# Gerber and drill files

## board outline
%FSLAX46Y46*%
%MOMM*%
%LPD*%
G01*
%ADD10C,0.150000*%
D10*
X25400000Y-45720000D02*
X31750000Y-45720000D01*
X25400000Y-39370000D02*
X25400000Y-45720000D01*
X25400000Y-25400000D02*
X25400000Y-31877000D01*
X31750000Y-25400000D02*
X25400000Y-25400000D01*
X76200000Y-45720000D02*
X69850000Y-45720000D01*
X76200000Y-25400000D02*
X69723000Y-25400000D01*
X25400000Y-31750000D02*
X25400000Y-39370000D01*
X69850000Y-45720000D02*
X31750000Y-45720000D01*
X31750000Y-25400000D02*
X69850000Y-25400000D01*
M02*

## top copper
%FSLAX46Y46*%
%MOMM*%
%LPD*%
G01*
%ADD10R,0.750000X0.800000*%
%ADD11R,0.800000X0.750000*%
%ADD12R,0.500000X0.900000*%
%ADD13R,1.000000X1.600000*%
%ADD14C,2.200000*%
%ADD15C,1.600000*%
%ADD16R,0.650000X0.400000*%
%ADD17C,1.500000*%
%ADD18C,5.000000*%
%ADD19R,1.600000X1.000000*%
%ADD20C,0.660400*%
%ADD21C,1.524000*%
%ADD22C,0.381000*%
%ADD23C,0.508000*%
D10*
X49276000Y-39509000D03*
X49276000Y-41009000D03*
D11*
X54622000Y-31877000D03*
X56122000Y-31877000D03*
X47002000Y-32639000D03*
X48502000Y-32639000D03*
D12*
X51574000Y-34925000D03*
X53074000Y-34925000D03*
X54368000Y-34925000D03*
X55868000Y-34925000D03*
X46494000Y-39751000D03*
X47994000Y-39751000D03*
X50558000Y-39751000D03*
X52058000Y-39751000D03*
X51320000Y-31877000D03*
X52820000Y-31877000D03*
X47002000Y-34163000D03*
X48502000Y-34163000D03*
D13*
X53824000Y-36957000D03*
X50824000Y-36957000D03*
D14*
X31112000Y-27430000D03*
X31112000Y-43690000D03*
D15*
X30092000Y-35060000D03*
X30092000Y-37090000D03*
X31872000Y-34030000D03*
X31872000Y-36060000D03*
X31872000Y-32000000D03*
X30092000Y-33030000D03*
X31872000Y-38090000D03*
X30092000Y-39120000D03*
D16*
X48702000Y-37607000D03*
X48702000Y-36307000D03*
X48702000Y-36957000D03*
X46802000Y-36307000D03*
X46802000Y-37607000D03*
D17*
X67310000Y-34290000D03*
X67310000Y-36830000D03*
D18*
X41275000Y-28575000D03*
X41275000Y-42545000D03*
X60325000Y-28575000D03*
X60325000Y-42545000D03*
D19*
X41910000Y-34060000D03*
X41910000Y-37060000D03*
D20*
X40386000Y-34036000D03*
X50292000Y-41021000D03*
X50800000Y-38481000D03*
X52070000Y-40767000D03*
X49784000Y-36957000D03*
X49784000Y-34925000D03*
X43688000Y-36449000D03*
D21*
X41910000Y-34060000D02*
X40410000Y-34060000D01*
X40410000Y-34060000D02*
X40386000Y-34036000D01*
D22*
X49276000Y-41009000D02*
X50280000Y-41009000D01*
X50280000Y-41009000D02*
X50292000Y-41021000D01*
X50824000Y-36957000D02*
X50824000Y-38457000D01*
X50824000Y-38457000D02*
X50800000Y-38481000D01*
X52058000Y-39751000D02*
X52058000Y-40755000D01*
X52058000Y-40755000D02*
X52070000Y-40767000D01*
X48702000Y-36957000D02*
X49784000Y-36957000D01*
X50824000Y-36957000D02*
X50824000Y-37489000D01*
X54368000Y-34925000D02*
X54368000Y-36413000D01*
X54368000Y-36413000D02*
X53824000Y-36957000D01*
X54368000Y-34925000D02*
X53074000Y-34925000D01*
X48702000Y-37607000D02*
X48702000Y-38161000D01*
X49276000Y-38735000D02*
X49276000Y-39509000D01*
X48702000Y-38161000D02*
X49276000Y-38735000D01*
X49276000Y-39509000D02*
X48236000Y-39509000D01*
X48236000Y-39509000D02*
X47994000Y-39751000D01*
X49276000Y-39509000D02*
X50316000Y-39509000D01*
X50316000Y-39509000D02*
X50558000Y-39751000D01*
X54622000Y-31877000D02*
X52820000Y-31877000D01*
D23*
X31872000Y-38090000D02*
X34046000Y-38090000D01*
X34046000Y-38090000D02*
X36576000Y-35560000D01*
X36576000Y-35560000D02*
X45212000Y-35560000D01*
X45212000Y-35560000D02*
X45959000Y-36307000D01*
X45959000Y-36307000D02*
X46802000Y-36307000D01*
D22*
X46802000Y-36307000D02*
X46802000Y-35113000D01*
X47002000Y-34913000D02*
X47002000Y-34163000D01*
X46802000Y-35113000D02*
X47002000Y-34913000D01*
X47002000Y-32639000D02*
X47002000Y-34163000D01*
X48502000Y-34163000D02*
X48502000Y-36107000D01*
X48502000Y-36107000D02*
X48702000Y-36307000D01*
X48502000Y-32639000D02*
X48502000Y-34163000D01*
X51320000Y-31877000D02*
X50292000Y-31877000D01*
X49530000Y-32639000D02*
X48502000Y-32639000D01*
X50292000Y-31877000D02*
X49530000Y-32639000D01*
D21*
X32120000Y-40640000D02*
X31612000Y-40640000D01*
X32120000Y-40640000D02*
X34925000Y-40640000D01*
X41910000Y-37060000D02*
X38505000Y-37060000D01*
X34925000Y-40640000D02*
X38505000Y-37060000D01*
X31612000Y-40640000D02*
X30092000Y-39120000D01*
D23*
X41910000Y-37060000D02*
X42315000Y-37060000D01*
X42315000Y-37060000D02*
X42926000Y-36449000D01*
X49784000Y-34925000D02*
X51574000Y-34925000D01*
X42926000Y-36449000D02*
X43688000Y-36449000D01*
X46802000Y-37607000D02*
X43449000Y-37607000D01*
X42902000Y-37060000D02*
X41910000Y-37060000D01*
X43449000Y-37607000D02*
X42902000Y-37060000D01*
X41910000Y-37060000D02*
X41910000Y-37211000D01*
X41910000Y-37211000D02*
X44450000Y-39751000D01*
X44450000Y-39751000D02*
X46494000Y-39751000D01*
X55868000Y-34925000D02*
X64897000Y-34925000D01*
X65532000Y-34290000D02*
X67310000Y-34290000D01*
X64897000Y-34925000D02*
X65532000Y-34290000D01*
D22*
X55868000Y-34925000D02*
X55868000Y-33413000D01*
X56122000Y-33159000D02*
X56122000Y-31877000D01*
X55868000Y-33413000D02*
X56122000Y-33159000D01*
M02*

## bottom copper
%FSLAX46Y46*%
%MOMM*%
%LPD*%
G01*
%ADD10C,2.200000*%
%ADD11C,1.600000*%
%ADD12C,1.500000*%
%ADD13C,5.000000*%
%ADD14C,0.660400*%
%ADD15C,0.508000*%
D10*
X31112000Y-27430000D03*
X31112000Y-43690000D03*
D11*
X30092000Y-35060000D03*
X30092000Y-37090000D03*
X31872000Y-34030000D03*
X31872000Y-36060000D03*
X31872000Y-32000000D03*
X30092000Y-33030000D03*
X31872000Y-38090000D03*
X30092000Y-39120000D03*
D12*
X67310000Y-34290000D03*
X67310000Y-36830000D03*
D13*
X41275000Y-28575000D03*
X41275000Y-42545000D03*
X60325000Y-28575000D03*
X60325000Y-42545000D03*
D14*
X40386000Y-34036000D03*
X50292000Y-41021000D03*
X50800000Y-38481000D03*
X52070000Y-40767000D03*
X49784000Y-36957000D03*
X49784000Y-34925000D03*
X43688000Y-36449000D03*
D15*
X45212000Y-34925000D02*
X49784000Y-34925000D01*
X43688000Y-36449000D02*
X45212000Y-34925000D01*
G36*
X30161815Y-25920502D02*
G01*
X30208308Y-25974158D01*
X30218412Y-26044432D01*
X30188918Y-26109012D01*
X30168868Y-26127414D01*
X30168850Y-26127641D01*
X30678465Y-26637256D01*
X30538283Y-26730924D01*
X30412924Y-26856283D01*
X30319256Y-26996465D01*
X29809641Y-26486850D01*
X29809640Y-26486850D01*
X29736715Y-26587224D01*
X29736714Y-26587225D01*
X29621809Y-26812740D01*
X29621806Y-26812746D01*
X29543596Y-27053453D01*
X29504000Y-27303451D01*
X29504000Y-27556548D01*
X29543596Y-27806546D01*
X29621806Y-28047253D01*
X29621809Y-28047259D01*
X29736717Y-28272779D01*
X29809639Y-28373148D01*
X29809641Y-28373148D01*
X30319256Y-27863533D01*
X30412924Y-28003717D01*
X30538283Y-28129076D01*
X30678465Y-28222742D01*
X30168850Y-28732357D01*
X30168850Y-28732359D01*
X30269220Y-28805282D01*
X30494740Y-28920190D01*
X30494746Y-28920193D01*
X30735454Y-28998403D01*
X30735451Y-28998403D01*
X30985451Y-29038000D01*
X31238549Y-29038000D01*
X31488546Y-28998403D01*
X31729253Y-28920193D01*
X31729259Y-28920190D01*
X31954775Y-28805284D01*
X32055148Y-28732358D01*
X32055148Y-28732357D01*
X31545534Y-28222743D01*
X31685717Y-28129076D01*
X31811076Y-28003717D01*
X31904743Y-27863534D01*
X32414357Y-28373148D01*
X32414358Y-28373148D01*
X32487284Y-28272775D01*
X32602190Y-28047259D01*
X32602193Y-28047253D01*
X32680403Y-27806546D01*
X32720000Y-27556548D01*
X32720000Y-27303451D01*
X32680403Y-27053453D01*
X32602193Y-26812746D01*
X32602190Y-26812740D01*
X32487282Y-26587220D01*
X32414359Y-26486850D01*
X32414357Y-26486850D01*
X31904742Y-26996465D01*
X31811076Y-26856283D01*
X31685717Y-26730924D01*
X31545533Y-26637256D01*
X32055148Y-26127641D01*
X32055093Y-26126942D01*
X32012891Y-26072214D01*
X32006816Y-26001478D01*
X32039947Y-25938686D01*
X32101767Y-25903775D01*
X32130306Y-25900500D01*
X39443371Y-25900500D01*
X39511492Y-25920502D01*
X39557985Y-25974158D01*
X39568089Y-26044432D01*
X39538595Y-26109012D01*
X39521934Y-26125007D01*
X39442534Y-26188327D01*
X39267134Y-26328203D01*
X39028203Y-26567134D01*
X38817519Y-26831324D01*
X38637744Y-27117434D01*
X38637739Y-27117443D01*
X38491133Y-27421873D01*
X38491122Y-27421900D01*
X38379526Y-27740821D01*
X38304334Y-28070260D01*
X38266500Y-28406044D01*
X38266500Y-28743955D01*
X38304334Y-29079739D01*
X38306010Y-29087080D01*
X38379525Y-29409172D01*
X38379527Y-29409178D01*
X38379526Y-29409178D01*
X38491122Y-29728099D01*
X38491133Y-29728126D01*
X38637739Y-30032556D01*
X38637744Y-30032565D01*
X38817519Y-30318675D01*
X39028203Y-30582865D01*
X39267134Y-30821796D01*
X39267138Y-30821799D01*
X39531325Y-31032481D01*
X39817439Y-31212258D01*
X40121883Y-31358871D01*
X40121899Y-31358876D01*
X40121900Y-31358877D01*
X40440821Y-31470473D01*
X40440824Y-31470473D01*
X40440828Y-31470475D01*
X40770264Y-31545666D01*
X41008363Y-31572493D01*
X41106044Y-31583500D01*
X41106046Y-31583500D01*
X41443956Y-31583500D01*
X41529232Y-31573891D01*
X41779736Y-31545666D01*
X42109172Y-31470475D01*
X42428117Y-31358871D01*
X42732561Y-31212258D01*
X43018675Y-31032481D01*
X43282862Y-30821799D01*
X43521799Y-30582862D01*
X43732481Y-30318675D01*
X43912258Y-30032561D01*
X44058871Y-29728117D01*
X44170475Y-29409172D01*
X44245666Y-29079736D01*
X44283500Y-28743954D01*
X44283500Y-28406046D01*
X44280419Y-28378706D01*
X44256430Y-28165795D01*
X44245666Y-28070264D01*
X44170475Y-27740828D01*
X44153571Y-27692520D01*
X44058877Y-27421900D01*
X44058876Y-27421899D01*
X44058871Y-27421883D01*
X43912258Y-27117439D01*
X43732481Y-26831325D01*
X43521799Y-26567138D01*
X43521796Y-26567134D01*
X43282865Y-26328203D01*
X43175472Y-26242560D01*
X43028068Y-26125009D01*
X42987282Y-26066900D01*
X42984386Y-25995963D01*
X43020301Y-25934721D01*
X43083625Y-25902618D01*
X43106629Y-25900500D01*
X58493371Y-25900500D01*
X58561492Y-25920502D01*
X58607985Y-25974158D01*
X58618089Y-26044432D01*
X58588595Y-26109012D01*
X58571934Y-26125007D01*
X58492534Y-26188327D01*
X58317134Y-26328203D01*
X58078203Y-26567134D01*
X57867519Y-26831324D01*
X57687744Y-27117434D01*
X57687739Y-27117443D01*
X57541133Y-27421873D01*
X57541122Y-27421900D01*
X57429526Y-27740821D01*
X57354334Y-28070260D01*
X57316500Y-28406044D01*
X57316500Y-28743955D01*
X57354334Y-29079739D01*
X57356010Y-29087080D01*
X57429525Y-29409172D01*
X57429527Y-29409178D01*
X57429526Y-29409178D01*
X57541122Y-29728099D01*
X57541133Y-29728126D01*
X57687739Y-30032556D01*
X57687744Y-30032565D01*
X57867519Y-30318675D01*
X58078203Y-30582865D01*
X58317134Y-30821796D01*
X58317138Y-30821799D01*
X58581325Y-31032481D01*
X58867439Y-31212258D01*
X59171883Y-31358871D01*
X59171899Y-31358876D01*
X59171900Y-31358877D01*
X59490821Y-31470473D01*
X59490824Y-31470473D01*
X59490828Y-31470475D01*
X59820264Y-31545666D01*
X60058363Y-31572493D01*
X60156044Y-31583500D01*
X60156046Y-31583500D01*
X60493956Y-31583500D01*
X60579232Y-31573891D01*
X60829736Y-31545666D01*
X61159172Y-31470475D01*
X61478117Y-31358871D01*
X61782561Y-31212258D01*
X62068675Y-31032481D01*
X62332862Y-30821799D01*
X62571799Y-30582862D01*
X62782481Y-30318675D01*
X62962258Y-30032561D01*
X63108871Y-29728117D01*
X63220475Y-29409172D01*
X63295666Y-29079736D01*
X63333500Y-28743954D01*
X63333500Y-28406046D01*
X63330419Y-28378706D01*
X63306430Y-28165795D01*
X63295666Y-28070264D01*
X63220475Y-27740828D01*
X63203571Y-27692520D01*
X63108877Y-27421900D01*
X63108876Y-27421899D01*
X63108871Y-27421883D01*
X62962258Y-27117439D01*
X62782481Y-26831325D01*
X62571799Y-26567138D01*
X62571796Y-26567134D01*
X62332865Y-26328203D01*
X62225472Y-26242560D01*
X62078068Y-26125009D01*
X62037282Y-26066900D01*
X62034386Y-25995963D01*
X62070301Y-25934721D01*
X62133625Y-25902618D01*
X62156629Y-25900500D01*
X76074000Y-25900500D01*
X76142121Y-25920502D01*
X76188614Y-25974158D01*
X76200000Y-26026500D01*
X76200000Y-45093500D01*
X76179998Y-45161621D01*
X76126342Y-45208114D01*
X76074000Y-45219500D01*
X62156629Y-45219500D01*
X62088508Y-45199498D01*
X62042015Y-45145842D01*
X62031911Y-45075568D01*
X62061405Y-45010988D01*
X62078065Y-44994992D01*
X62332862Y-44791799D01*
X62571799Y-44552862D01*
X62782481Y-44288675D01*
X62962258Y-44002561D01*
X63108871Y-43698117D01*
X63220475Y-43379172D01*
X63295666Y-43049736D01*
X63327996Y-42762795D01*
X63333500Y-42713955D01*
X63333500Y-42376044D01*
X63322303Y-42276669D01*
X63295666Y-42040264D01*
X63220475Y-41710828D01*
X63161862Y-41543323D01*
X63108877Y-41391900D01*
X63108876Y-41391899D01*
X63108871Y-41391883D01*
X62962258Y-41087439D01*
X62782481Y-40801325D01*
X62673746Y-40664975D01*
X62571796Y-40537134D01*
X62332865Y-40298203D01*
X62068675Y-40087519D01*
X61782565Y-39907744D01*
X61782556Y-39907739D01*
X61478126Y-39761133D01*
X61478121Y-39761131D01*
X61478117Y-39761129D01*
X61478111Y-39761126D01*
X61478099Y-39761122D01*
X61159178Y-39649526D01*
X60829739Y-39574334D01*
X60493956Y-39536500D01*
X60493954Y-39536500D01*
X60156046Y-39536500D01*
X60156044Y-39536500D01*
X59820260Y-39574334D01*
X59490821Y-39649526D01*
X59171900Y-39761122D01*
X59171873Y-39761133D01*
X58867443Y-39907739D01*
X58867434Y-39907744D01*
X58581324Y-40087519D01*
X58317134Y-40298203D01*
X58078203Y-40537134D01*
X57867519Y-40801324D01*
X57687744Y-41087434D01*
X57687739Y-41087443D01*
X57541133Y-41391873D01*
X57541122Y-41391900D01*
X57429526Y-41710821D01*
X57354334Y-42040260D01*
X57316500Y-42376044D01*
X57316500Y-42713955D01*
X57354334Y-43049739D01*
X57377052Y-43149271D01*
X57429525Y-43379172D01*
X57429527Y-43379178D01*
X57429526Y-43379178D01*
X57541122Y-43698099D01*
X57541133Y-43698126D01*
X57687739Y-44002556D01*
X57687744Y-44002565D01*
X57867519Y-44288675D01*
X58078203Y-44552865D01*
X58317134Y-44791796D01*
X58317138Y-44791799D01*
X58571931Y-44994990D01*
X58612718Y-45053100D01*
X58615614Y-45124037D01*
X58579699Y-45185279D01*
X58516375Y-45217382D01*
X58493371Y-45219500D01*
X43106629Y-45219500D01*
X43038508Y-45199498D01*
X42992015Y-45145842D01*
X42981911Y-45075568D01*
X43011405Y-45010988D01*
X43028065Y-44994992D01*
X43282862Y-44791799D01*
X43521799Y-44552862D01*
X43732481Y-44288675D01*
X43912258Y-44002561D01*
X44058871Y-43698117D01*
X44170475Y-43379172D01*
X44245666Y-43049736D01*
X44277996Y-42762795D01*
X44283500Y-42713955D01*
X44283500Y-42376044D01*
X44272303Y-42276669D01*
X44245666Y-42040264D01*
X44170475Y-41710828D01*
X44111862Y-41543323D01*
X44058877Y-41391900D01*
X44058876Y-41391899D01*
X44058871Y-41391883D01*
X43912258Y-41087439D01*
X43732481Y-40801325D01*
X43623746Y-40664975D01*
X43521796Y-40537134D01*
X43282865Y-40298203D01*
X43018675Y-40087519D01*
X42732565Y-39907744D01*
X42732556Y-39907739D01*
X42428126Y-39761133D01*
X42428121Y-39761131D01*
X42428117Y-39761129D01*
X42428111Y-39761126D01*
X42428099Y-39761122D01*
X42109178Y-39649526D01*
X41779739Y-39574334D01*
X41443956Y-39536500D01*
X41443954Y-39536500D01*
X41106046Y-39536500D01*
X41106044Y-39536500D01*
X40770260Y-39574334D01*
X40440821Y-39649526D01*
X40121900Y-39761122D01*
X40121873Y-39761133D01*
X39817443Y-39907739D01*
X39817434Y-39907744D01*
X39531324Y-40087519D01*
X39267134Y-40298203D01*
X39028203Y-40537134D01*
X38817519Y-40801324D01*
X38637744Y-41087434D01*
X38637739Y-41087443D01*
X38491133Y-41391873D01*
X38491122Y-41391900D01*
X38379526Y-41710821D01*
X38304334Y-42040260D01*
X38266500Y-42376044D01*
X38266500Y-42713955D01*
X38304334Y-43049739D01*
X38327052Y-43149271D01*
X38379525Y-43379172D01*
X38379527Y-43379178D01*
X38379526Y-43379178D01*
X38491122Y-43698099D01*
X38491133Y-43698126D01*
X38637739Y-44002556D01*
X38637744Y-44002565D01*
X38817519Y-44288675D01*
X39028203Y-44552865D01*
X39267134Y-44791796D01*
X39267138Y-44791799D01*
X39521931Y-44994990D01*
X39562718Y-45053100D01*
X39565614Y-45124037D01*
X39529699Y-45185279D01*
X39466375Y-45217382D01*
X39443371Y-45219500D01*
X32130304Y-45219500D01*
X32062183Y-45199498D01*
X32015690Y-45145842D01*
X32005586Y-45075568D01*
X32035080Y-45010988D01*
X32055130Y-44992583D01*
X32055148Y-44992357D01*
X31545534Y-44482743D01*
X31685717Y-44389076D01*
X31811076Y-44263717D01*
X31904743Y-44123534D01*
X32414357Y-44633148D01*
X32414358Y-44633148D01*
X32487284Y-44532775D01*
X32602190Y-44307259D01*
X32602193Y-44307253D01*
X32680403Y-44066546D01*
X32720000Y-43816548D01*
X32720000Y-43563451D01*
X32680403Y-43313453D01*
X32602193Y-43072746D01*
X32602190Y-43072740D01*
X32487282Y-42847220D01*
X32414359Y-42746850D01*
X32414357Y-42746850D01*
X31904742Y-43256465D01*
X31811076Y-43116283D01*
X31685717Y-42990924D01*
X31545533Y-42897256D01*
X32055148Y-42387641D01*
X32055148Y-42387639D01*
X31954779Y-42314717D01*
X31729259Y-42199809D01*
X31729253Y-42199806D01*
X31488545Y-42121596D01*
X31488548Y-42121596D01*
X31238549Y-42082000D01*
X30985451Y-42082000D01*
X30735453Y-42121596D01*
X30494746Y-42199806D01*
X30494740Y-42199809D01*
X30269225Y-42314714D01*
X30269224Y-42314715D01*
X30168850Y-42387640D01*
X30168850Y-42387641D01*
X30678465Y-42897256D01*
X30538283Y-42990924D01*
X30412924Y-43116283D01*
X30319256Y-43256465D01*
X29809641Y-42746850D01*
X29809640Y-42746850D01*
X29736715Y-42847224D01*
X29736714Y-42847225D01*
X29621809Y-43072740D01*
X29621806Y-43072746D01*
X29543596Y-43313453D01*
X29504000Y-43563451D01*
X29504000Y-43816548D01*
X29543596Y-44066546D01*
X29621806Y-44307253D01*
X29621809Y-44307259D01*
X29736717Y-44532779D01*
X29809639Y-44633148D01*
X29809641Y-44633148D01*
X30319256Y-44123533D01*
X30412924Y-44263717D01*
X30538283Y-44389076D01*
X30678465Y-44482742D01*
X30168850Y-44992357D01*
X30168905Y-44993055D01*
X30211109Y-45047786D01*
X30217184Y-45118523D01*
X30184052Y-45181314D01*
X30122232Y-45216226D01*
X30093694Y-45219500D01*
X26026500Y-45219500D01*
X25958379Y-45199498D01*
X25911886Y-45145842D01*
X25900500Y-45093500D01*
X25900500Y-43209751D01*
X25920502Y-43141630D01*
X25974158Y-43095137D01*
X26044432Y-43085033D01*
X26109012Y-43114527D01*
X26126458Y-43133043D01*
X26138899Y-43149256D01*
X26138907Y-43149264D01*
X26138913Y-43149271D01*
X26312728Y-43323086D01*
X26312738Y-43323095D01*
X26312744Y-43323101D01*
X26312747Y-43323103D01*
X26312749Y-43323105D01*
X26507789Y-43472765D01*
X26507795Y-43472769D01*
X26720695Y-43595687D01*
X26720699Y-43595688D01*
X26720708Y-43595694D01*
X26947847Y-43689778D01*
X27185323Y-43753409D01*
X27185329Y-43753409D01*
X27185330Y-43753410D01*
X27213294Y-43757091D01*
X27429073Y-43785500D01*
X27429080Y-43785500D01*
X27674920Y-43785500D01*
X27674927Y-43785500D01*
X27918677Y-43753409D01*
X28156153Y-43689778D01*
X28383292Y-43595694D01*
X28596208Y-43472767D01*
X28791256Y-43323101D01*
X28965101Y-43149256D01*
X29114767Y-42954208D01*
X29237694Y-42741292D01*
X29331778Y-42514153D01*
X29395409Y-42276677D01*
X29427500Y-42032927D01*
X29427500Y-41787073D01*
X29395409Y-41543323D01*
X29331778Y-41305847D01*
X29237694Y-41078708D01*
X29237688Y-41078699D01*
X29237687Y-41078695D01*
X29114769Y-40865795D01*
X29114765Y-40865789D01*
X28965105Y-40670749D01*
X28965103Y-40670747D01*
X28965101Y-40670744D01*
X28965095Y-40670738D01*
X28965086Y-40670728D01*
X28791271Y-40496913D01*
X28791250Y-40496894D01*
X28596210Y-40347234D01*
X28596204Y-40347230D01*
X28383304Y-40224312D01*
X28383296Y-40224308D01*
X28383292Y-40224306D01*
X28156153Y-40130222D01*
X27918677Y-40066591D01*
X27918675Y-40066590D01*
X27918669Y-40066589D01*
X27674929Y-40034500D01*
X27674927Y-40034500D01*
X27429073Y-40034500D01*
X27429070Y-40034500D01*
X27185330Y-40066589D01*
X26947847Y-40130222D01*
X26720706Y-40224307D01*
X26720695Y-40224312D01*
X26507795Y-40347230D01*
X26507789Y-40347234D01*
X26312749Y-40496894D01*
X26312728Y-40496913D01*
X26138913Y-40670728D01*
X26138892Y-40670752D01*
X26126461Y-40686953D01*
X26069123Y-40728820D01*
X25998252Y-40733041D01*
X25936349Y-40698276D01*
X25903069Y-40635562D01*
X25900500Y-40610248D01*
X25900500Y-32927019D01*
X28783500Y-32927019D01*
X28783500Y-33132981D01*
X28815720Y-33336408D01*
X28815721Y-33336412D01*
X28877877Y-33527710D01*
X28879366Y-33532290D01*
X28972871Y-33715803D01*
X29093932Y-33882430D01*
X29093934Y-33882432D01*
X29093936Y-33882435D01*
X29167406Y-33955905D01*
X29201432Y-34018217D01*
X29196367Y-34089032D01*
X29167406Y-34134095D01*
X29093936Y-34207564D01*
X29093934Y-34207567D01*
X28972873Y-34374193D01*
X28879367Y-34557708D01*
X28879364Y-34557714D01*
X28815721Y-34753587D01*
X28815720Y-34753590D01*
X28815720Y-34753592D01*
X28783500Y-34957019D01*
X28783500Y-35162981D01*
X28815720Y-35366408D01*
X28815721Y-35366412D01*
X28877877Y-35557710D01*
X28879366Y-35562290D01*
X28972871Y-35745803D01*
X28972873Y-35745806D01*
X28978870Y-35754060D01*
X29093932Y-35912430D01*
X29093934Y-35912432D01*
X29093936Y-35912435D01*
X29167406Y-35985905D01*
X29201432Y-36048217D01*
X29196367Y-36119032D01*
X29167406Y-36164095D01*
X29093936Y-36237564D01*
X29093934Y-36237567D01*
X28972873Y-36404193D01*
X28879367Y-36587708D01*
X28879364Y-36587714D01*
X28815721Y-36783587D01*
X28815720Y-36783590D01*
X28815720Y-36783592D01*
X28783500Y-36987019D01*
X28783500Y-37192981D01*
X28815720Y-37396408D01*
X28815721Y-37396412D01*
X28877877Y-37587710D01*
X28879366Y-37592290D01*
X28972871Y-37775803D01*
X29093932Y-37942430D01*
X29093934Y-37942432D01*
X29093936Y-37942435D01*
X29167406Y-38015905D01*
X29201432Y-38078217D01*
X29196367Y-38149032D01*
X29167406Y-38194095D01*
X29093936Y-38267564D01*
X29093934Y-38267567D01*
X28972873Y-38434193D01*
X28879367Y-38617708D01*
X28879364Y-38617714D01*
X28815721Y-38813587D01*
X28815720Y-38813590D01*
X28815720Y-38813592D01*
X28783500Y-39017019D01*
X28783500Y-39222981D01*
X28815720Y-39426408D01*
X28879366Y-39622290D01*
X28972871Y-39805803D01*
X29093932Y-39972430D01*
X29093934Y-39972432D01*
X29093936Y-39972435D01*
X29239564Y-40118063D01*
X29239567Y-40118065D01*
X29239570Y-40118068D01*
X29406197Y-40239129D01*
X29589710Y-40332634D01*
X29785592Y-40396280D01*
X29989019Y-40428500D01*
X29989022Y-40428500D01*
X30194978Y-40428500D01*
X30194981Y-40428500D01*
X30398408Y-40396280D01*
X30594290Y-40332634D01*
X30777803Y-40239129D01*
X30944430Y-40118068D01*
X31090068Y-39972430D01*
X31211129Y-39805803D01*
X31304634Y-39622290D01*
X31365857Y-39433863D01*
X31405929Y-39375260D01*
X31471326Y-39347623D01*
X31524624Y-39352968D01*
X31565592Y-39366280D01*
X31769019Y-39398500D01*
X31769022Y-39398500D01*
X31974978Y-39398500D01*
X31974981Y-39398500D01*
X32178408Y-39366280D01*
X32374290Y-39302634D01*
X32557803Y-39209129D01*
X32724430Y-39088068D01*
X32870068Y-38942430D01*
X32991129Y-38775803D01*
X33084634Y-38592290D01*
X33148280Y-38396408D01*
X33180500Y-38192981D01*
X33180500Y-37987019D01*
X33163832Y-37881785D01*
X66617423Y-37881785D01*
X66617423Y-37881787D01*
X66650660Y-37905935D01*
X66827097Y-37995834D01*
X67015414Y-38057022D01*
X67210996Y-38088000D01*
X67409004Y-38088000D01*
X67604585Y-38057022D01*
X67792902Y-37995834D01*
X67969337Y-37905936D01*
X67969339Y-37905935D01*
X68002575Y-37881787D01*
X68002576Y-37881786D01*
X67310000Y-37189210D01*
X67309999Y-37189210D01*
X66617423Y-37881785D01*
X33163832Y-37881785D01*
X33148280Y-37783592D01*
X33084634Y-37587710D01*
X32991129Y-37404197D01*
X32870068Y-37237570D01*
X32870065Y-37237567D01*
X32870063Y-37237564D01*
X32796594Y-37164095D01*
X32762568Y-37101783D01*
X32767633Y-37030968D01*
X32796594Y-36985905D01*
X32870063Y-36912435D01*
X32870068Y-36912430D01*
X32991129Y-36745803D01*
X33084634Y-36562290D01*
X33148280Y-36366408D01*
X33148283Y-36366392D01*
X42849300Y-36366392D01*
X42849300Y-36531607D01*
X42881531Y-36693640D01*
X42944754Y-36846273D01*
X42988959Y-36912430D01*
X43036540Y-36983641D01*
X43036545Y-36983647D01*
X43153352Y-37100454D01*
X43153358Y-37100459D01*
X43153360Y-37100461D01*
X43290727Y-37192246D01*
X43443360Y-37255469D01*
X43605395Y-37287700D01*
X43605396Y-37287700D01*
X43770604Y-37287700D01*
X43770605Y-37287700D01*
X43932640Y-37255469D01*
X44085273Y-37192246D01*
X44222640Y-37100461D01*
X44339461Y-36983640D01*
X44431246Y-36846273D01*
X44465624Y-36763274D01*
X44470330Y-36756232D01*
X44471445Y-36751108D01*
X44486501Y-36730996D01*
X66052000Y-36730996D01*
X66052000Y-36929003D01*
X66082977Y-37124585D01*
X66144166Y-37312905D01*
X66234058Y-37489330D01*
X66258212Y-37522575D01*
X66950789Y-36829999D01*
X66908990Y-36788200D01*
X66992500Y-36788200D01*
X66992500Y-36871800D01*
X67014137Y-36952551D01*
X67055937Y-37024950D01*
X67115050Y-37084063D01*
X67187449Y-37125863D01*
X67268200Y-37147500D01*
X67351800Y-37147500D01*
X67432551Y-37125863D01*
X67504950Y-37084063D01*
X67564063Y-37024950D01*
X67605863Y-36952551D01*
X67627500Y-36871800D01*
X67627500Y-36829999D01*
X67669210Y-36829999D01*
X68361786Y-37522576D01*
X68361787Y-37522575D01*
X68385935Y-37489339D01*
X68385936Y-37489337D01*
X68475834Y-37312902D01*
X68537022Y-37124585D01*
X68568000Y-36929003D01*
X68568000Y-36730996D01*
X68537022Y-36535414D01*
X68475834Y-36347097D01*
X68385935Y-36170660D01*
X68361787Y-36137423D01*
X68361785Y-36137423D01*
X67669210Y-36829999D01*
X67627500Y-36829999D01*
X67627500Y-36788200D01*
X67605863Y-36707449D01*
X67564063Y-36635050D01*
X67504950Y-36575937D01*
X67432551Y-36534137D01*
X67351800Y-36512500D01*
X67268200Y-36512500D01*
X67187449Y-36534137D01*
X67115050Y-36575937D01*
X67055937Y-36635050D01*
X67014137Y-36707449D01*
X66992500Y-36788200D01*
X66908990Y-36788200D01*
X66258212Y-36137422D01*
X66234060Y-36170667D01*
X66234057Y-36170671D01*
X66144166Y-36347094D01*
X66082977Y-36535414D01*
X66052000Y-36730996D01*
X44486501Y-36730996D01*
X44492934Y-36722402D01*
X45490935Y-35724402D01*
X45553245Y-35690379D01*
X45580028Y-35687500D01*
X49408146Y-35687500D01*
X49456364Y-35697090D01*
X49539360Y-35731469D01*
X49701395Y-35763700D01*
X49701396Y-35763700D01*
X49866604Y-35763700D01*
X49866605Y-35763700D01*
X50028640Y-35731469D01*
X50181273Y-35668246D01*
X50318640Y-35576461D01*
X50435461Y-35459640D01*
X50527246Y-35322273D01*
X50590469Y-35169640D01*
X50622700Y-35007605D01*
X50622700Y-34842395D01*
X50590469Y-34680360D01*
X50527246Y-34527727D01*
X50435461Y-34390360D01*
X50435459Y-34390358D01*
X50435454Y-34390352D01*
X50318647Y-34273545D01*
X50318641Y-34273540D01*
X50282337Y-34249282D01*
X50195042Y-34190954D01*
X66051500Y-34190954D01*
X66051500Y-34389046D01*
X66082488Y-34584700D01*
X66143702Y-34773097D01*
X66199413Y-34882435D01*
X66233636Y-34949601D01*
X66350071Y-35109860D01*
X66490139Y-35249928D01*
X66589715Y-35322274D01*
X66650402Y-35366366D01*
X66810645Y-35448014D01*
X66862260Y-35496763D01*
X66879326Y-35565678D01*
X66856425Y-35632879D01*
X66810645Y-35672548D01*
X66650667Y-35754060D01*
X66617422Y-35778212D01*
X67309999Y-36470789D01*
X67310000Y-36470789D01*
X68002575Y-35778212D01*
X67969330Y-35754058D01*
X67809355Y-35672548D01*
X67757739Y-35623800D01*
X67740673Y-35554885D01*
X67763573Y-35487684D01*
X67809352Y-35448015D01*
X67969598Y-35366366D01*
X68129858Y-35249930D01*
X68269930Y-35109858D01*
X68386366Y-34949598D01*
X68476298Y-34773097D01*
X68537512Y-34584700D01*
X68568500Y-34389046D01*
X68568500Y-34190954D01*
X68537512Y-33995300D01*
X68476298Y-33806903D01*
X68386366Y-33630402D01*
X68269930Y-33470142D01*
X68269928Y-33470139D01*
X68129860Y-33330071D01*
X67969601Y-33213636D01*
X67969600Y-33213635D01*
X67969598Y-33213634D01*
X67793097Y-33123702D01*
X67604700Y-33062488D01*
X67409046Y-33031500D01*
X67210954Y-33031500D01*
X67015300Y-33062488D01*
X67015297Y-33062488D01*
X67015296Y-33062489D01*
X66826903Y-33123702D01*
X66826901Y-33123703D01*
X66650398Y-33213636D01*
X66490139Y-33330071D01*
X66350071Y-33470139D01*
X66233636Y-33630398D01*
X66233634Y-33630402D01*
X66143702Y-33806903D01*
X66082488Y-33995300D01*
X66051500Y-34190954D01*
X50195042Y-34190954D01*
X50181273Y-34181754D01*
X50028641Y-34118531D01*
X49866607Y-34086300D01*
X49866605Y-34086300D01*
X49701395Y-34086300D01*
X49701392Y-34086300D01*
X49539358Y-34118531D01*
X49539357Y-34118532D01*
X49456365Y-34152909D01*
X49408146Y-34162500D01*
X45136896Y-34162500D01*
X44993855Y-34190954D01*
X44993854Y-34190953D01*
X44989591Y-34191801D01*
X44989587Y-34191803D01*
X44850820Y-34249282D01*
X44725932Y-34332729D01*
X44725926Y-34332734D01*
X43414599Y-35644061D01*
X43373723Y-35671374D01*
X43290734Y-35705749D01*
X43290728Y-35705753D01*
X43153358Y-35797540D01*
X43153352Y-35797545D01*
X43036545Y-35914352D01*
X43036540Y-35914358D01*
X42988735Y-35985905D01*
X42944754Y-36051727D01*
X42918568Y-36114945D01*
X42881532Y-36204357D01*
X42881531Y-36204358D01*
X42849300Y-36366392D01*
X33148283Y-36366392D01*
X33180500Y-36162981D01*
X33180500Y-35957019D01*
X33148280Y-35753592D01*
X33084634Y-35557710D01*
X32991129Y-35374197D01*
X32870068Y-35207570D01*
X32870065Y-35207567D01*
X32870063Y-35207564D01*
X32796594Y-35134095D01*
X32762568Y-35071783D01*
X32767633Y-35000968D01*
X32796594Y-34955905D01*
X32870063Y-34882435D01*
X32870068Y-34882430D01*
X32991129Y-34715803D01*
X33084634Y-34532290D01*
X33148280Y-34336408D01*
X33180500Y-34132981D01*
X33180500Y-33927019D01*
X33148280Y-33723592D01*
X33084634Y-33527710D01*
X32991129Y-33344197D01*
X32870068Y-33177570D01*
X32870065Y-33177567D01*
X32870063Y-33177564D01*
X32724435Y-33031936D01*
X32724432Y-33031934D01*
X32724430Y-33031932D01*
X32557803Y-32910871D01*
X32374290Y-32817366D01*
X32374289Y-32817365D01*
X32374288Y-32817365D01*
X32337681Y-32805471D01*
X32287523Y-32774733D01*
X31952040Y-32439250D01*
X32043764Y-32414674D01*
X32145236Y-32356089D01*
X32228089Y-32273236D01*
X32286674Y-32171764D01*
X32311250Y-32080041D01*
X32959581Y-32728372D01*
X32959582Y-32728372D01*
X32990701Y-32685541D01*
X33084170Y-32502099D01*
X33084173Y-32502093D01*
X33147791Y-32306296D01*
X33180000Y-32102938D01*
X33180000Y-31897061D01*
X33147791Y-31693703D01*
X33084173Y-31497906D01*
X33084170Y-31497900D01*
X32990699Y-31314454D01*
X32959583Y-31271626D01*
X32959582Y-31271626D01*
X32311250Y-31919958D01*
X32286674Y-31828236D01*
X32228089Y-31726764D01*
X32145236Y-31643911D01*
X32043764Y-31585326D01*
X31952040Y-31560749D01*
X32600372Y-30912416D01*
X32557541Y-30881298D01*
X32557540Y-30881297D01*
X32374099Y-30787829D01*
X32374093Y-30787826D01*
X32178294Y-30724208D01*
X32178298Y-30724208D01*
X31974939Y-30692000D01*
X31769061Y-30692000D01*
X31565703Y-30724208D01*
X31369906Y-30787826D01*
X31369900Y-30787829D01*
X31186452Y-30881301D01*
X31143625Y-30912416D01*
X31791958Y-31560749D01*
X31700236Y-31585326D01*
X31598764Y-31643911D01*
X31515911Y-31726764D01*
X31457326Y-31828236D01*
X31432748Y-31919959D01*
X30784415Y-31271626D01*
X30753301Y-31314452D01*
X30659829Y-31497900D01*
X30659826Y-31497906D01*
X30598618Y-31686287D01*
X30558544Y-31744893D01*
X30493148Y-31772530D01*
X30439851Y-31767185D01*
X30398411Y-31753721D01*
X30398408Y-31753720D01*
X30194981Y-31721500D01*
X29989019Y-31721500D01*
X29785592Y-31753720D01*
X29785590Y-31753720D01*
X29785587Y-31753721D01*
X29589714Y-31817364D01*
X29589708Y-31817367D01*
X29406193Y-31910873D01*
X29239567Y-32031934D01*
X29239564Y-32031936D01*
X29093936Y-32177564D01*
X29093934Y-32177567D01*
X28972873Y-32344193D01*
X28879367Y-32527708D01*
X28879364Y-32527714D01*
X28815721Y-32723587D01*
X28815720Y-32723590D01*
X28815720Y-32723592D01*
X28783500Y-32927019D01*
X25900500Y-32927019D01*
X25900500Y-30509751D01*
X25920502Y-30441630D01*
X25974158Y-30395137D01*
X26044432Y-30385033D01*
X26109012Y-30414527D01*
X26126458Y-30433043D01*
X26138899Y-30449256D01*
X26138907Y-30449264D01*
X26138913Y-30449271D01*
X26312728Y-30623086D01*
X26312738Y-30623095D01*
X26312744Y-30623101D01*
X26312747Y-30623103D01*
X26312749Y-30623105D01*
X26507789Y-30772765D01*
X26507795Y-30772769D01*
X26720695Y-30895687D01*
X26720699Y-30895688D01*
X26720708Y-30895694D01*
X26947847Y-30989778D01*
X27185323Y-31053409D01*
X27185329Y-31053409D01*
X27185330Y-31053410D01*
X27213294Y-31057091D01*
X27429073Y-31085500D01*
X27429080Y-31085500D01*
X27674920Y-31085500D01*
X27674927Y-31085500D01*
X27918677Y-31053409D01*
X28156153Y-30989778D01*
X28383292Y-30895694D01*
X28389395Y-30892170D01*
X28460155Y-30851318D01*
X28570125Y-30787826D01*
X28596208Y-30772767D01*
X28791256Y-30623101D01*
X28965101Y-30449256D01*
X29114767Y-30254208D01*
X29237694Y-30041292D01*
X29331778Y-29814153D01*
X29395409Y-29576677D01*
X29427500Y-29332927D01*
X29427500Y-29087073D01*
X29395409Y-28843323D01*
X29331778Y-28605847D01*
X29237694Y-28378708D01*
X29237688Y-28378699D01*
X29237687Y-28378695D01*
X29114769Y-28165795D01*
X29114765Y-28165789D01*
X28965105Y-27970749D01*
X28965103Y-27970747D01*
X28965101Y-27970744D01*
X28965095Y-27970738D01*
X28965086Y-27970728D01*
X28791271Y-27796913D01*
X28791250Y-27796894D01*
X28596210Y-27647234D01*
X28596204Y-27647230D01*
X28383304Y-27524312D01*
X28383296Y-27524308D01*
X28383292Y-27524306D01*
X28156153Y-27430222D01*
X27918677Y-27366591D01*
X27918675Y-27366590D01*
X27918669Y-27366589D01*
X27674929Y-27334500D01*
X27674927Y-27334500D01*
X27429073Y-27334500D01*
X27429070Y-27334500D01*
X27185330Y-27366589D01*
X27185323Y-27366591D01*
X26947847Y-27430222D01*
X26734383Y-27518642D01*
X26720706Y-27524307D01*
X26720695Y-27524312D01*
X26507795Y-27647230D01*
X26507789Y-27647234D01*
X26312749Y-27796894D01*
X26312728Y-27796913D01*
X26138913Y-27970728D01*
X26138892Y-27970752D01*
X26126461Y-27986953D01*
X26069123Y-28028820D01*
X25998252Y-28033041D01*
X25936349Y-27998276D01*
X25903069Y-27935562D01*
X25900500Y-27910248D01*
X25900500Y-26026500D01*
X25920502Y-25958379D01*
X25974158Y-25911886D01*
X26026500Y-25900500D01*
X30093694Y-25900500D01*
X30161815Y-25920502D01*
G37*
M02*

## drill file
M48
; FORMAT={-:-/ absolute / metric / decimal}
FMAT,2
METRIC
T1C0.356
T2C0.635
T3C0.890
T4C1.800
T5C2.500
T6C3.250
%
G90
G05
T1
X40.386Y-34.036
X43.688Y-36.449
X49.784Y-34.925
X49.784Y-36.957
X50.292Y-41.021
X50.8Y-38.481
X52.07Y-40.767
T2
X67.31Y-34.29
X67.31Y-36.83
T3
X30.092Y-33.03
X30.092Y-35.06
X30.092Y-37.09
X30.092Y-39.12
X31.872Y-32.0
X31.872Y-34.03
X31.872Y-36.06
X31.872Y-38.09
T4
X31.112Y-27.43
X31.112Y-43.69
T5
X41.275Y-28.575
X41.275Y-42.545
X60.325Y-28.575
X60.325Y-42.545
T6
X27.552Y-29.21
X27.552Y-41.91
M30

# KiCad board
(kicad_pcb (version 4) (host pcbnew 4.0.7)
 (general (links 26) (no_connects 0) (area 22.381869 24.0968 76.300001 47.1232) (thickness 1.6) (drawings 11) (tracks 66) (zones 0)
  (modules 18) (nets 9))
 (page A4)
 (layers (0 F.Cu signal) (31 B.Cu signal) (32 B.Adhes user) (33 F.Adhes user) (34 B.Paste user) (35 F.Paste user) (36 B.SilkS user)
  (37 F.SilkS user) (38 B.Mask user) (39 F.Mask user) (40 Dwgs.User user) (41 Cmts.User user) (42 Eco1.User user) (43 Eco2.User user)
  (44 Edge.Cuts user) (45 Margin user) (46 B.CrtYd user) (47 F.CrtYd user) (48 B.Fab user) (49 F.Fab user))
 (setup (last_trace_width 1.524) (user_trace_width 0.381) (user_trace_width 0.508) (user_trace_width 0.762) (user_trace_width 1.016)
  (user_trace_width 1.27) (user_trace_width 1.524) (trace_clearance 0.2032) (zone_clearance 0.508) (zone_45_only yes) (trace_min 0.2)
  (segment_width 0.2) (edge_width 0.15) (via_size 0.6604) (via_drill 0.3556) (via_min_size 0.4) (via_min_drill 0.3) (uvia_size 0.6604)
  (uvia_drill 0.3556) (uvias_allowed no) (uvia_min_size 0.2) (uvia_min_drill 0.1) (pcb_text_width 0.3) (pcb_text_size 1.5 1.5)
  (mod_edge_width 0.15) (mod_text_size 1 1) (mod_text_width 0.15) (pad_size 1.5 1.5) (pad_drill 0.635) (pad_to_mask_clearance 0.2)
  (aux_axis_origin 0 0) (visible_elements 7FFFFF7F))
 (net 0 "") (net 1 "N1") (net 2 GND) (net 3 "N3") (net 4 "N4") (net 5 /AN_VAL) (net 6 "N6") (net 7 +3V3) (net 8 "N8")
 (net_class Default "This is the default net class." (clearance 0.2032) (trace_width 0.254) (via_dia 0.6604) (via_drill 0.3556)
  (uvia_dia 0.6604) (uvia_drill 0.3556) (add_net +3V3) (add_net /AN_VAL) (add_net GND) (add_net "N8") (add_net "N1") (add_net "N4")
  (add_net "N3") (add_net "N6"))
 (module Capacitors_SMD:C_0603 (layer F.Cu) (at 49.276 40.259 90)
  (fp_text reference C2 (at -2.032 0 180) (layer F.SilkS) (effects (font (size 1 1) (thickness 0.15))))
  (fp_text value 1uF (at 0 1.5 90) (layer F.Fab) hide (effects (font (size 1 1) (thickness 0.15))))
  (pad 2 smd rect (at 0.75 0 90) (size 0.8 0.75) (layers F.Cu F.Paste F.Mask) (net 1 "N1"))
  (pad 1 smd rect (at -0.75 0 90) (size 0.8 0.75) (layers F.Cu F.Paste F.Mask) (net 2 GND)))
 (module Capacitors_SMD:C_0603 (layer F.Cu) (at 55.372 31.877 180)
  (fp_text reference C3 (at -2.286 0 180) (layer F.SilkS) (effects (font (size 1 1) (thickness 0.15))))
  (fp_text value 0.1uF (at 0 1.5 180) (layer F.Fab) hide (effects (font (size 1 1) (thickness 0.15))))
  (pad 2 smd rect (at 0.75 0 180) (size 0.8 0.75) (layers F.Cu F.Paste F.Mask) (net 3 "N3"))
  (pad 1 smd rect (at -0.75 0 180) (size 0.8 0.75) (layers F.Cu F.Paste F.Mask) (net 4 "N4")))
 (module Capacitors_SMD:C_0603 (layer F.Cu) (at 47.752 32.639 180)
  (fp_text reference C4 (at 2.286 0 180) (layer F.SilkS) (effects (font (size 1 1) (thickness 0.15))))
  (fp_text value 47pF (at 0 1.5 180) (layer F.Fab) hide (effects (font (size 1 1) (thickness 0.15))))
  (pad 2 smd rect (at 0.75 0 180) (size 0.8 0.75) (layers F.Cu F.Paste F.Mask) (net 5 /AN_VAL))
  (pad 1 smd rect (at -0.75 0 180) (size 0.8 0.75) (layers F.Cu F.Paste F.Mask) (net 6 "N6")))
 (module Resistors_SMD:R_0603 (layer F.Cu) (at 52.324 34.925)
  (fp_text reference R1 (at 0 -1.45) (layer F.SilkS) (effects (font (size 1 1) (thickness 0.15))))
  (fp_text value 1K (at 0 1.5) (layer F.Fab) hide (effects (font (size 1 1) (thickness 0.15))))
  (pad 1 smd rect (at -0.75 0) (size 0.5 0.9) (layers F.Cu F.Paste F.Mask) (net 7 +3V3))
  (pad 2 smd rect (at 0.75 0) (size 0.5 0.9) (layers F.Cu F.Paste F.Mask) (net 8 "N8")))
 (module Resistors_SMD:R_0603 (layer F.Cu) (at 55.118 34.925)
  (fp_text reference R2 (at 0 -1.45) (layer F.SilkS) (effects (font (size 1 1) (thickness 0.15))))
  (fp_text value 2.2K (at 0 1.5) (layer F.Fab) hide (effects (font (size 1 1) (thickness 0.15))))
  (pad 1 smd rect (at -0.75 0) (size 0.5 0.9) (layers F.Cu F.Paste F.Mask) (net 8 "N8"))
  (pad 2 smd rect (at 0.75 0) (size 0.5 0.9) (layers F.Cu F.Paste F.Mask) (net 4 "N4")))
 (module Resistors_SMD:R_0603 (layer F.Cu) (at 47.244 39.751)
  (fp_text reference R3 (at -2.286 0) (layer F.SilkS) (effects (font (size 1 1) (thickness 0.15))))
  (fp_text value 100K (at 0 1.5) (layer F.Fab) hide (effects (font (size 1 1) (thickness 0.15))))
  (pad 1 smd rect (at -0.75 0) (size 0.5 0.9) (layers F.Cu F.Paste F.Mask) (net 7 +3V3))
  (pad 2 smd rect (at 0.75 0) (size 0.5 0.9) (layers F.Cu F.Paste F.Mask) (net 1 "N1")))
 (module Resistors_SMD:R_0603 (layer F.Cu) (at 51.308 39.751)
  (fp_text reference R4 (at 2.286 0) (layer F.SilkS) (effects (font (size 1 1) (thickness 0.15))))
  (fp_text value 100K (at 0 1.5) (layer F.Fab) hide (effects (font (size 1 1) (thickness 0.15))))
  (pad 1 smd rect (at -0.75 0) (size 0.5 0.9) (layers F.Cu F.Paste F.Mask) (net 1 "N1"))
  (pad 2 smd rect (at 0.75 0) (size 0.5 0.9) (layers F.Cu F.Paste F.Mask) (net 2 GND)))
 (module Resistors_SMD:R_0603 (layer F.Cu) (at 52.07 31.877)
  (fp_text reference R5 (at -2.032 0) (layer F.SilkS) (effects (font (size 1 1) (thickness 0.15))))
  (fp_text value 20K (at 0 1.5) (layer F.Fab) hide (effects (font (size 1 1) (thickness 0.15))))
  (pad 1 smd rect (at -0.75 0) (size 0.5 0.9) (layers F.Cu F.Paste F.Mask) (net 6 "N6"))
  (pad 2 smd rect (at 0.75 0) (size 0.5 0.9) (layers F.Cu F.Paste F.Mask) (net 3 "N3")))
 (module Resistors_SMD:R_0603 (layer F.Cu) (at 47.752 34.163)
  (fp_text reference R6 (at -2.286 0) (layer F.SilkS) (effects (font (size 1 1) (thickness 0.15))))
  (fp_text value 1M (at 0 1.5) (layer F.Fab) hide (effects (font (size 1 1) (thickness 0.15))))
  (pad 1 smd rect (at -0.75 0) (size 0.5 0.9) (layers F.Cu F.Paste F.Mask) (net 5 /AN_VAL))
  (pad 2 smd rect (at 0.75 0) (size 0.5 0.9) (layers F.Cu F.Paste F.Mask) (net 6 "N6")))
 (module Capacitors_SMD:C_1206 (layer F.Cu) (at 52.324 36.957 180)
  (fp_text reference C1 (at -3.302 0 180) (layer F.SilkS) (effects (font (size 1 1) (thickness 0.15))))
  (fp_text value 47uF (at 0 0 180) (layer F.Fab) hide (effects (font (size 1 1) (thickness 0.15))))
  (pad 1 smd rect (at -1.5 0 180) (size 1 1.6) (layers F.Cu F.Paste F.Mask) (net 8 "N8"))
  (pad 2 smd rect (at 1.5 0 180) (size 1 1.6) (layers F.Cu F.Paste F.Mask) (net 2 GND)))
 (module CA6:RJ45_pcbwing (layer F.Cu) (at 29.972 35.56 270)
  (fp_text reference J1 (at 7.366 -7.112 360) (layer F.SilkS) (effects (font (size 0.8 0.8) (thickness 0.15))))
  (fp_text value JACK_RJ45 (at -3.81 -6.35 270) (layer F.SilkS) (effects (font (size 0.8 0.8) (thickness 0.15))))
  (pad 8 thru_hole circle (at -8.13 -1.14 270) (size 2.2 2.2) (drill 1.8) (layers *.Cu *.Mask F.SilkS) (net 2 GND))
  (pad 8 thru_hole circle (at 8.13 -1.14 270) (size 2.2 2.2) (drill 1.8) (layers *.Cu *.Mask F.SilkS) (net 2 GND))
  (pad "" np_thru_hole circle (at -6.35 2.42 270) (size 3.25 3.25) (drill 3.25) (layers *.Cu *.Mask F.SilkS))
  (pad "" np_thru_hole circle (at 6.35 2.42 270) (size 3.25 3.25) (drill 3.25) (layers *.Cu *.Mask F.SilkS))
  (pad 5 thru_hole circle (at -0.5 -0.12 270) (size 1.6 1.6) (drill 0.89) (layers *.Cu *.Mask F.SilkS))
  (pad 3 thru_hole circle (at 1.53 -0.12 270) (size 1.6 1.6) (drill 0.89) (layers *.Cu *.Mask F.SilkS))
  (pad 6 thru_hole circle (at -1.53 -1.9 270) (size 1.6 1.6) (drill 0.89) (layers *.Cu *.Mask F.SilkS))
  (pad 4 thru_hole circle (at 0.5 -1.9 270) (size 1.6 1.6) (drill 0.89) (layers *.Cu *.Mask F.SilkS))
  (pad 8 thru_hole circle (at -3.56 -1.9 270) (size 1.6 1.6) (drill 0.89) (layers *.Cu *.Mask F.SilkS) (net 2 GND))
  (pad 7 thru_hole circle (at -2.53 -0.12 270) (size 1.6 1.6) (drill 0.89) (layers *.Cu *.Mask F.SilkS))
  (pad 2 thru_hole circle (at 2.53 -1.9 270) (size 1.6 1.6) (drill 0.89) (layers *.Cu *.Mask F.SilkS) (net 5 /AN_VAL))
  (pad 1 thru_hole circle (at 3.56 -0.12 270) (size 1.6 1.6) (drill 0.89) (layers *.Cu *.Mask F.SilkS) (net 7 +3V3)))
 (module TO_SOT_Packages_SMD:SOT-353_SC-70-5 (layer F.Cu) (at 47.752 36.957 180)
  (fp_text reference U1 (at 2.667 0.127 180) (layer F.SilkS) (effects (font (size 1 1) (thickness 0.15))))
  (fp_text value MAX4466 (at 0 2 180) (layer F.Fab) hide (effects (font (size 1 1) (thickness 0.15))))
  (pad 1 smd rect (at -0.95 -0.65 180) (size 0.65 0.4) (layers F.Cu F.Paste F.Mask) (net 1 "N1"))
  (pad 3 smd rect (at -0.95 0.65 180) (size 0.65 0.4) (layers F.Cu F.Paste F.Mask) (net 6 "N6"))
  (pad 2 smd rect (at -0.95 0 180) (size 0.65 0.4) (layers F.Cu F.Paste F.Mask) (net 2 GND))
  (pad 4 smd rect (at 0.95 0.65 180) (size 0.65 0.4) (layers F.Cu F.Paste F.Mask) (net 5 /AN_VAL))
  (pad 5 smd rect (at 0.95 -0.65 180) (size 0.65 0.4) (layers F.Cu F.Paste F.Mask) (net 7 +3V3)))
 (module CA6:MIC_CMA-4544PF (layer F.Cu) (at 69.31 35.56 180)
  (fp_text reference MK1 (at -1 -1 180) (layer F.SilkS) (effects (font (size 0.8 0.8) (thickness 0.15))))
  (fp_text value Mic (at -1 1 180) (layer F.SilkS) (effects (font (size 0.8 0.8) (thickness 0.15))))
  (pad 1 thru_hole circle (at 2 1.27 180) (size 1.5 1.5) (drill 0.635) (layers *.Cu *.Mask) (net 4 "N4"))
  (pad 2 thru_hole circle (at 2 -1.27 180) (size 1.5 1.5) (drill 0.635) (layers *.Cu *.Mask) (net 2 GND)))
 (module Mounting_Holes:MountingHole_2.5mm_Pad (layer F.Cu) (at 41.275 28.575)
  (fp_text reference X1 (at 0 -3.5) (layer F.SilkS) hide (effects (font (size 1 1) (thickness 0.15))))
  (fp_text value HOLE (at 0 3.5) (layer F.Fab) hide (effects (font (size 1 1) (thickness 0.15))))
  (pad 1 thru_hole circle (at 0 0) (size 5 5) (drill 2.5) (layers *.Cu *.Mask)))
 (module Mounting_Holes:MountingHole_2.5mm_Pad (layer F.Cu) (at 41.275 42.545)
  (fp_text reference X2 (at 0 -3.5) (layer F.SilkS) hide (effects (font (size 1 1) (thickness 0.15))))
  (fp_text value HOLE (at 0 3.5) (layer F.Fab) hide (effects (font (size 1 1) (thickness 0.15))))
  (pad 1 thru_hole circle (at 0 0) (size 5 5) (drill 2.5) (layers *.Cu *.Mask)))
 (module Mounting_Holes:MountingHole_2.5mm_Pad (layer F.Cu) (at 60.325 28.575)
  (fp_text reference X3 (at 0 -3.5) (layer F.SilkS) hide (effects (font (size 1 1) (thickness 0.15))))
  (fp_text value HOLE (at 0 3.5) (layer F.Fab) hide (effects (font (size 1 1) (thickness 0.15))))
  (pad 1 thru_hole circle (at 0 0) (size 5 5) (drill 2.5) (layers *.Cu *.Mask)))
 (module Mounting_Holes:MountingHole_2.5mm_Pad (layer F.Cu) (at 60.325 42.545)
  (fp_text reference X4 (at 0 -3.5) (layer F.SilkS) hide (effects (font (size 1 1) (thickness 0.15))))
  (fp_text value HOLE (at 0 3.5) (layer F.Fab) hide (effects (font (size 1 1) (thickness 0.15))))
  (pad 1 thru_hole circle (at 0 0) (size 5 5) (drill 2.5) (layers *.Cu *.Mask)))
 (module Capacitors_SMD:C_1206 (layer F.Cu) (at 41.91 35.56 270)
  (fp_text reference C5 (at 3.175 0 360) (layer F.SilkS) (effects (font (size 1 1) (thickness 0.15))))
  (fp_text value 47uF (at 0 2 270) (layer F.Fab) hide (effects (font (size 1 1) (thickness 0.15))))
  (pad 1 smd rect (at -1.5 0 270) (size 1 1.6) (layers F.Cu F.Paste F.Mask) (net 2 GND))
  (pad 2 smd rect (at 1.5 0 270) (size 1 1.6) (layers F.Cu F.Paste F.Mask) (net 7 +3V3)))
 (gr_line (start 25.4 45.72) (end 31.75 45.72) (angle 90) (layer Edge.Cuts) (width 0.15))
 (gr_line (start 25.4 39.37) (end 25.4 45.72) (angle 90) (layer Edge.Cuts) (width 0.15))
 (gr_line (start 25.4 25.4) (end 25.4 31.877) (angle 90) (layer Edge.Cuts) (width 0.15))
 (gr_line (start 31.75 25.4) (end 25.4 25.4) (angle 90) (layer Edge.Cuts) (width 0.15))
 (gr_line (start 76.2 45.72) (end 69.85 45.72) (angle 90) (layer Edge.Cuts) (width 0.15))
 (gr_line (start 76.2 25.4) (end 69.723 25.4) (angle 90) (layer Edge.Cuts) (width 0.15))
 (gr_line (start 25.4 31.75) (end 25.4 39.37) (angle 90) (layer Edge.Cuts) (width 0.15))
 (gr_line (start 69.85 45.72) (end 31.75 45.72) (angle 90) (layer Edge.Cuts) (width 0.15))
 (gr_line (start 31.75 25.4) (end 69.85 25.4) (angle 90) (layer Edge.Cuts) (width 0.15))
 (segment (start 41.91 34.06) (end 40.41 34.06) (width 1.524) (layer F.Cu) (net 2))
 (segment (start 40.41 34.06) (end 40.386 34.036) (width 1.524) (layer F.Cu) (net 2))
 (via (at 40.386 34.036) (size 0.6604) (drill 0.3556) (layers F.Cu B.Cu) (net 2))
 (segment (start 49.276 41.009) (end 50.28 41.009) (width 0.381) (layer F.Cu) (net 2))
 (via (at 50.292 41.021) (size 0.6604) (drill 0.3556) (layers F.Cu B.Cu) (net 2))
 (segment (start 50.28 41.009) (end 50.292 41.021) (width 0.381) (layer F.Cu) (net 2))
 (segment (start 50.824 36.957) (end 50.824 38.457) (width 0.381) (layer F.Cu) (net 2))
 (via (at 50.8 38.481) (size 0.6604) (drill 0.3556) (layers F.Cu B.Cu) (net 2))
 (segment (start 50.824 38.457) (end 50.8 38.481) (width 0.381) (layer F.Cu) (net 2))
 (segment (start 52.058 39.751) (end 52.058 40.755) (width 0.381) (layer F.Cu) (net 2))
 (via (at 52.07 40.767) (size 0.6604) (drill 0.3556) (layers F.Cu B.Cu) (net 2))
 (segment (start 52.058 40.755) (end 52.07 40.767) (width 0.381) (layer F.Cu) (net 2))
 (segment (start 48.702 36.957) (end 49.784 36.957) (width 0.381) (layer F.Cu) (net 2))
 (via (at 49.784 36.957) (size 0.6604) (drill 0.3556) (layers F.Cu B.Cu) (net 2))
 (segment (start 50.824 36.957) (end 50.824 37.489) (width 0.381) (layer F.Cu) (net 2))
 (segment (start 54.368 34.925) (end 54.368 36.413) (width 0.381) (layer F.Cu) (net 8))
 (segment (start 54.368 36.413) (end 53.824 36.957) (width 0.381) (layer F.Cu) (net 8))
 (segment (start 54.368 34.925) (end 53.074 34.925) (width 0.381) (layer F.Cu) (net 8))
 (segment (start 48.702 37.607) (end 48.702 38.161) (width 0.381) (layer F.Cu) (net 1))
 (segment (start 49.276 38.735) (end 49.276 39.509) (width 0.381) (layer F.Cu) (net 1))
 (segment (start 48.702 38.161) (end 49.276 38.735) (width 0.381) (layer F.Cu) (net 1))
 (segment (start 49.276 39.509) (end 48.236 39.509) (width 0.381) (layer F.Cu) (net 1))
 (segment (start 48.236 39.509) (end 47.994 39.751) (width 0.381) (layer F.Cu) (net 1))
 (segment (start 49.276 39.509) (end 50.316 39.509) (width 0.381) (layer F.Cu) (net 1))
 (segment (start 50.316 39.509) (end 50.558 39.751) (width 0.381) (layer F.Cu) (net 1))
 (segment (start 54.622 31.877) (end 52.82 31.877) (width 0.381) (layer F.Cu) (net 3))
 (segment (start 31.872 38.09) (end 34.046 38.09) (width 0.508) (layer F.Cu) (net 5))
 (segment (start 34.046 38.09) (end 36.576 35.56) (width 0.508) (layer F.Cu) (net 5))
 (segment (start 36.576 35.56) (end 45.212 35.56) (width 0.508) (layer F.Cu) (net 5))
 (segment (start 45.212 35.56) (end 45.959 36.307) (width 0.508) (layer F.Cu) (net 5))
 (segment (start 45.959 36.307) (end 46.802 36.307) (width 0.508) (layer F.Cu) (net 5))
 (segment (start 46.802 36.307) (end 46.802 35.113) (width 0.381) (layer F.Cu) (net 5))
 (segment (start 47.002 34.913) (end 47.002 34.163) (width 0.381) (layer F.Cu) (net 5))
 (segment (start 46.802 35.113) (end 47.002 34.913) (width 0.381) (layer F.Cu) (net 5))
 (segment (start 47.002 32.639) (end 47.002 34.163) (width 0.381) (layer F.Cu) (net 5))
 (segment (start 48.502 34.163) (end 48.502 36.107) (width 0.381) (layer F.Cu) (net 6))
 (segment (start 48.502 36.107) (end 48.702 36.307) (width 0.381) (layer F.Cu) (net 6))
 (segment (start 48.502 32.639) (end 48.502 34.163) (width 0.381) (layer F.Cu) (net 6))
 (segment (start 51.32 31.877) (end 50.292 31.877) (width 0.381) (layer F.Cu) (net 6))
 (segment (start 49.53 32.639) (end 48.502 32.639) (width 0.381) (layer F.Cu) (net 6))
 (segment (start 50.292 31.877) (end 49.53 32.639) (width 0.381) (layer F.Cu) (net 6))
 (segment (start 32.12 40.64) (end 31.612 40.64) (width 1.524) (layer F.Cu) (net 7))
 (segment (start 32.12 40.64) (end 34.925 40.64) (width 1.524) (layer F.Cu) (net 7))
 (segment (start 41.91 37.06) (end 38.505 37.06) (width 1.524) (layer F.Cu) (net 7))
 (segment (start 34.925 40.64) (end 38.505 37.06) (width 1.524) (layer F.Cu) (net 7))
 (segment (start 31.612 40.64) (end 30.092 39.12) (width 1.524) (layer F.Cu) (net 7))
 (segment (start 41.91 37.06) (end 42.315 37.06) (width 0.508) (layer F.Cu) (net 7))
 (segment (start 42.315 37.06) (end 42.926 36.449) (width 0.508) (layer F.Cu) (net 7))
 (segment (start 49.784 34.925) (end 51.574 34.925) (width 0.508) (layer F.Cu) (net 7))
 (via (at 49.784 34.925) (size 0.6604) (drill 0.3556) (layers F.Cu B.Cu) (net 7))
 (segment (start 45.212 34.925) (end 49.784 34.925) (width 0.508) (layer B.Cu) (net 7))
 (segment (start 43.688 36.449) (end 45.212 34.925) (width 0.508) (layer B.Cu) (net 7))
 (via (at 43.688 36.449) (size 0.6604) (drill 0.3556) (layers F.Cu B.Cu) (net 7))
 (segment (start 42.926 36.449) (end 43.688 36.449) (width 0.508) (layer F.Cu) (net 7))
 (segment (start 46.802 37.607) (end 43.449 37.607) (width 0.508) (layer F.Cu) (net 7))
 (segment (start 42.902 37.06) (end 41.91 37.06) (width 0.508) (layer F.Cu) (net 7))
 (segment (start 43.449 37.607) (end 42.902 37.06) (width 0.508) (layer F.Cu) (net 7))
 (segment (start 41.91 37.06) (end 41.91 37.211) (width 0.508) (layer F.Cu) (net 7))
 (segment (start 41.91 37.211) (end 44.45 39.751) (width 0.508) (layer F.Cu) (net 7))
 (segment (start 44.45 39.751) (end 46.494 39.751) (width 0.508) (layer F.Cu) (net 7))
 (segment (start 55.868 34.925) (end 64.897 34.925) (width 0.508) (layer F.Cu) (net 4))
 (segment (start 65.532 34.29) (end 67.31 34.29) (width 0.508) (layer F.Cu) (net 4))
 (segment (start 64.897 34.925) (end 65.532 34.29) (width 0.508) (layer F.Cu) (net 4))
 (segment (start 55.868 34.925) (end 55.868 33.413) (width 0.381) (layer F.Cu) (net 4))
 (segment (start 56.122 33.159) (end 56.122 31.877) (width 0.381) (layer F.Cu) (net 4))
 (segment (start 55.868 33.413) (end 56.122 33.159) (width 0.381) (layer F.Cu) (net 4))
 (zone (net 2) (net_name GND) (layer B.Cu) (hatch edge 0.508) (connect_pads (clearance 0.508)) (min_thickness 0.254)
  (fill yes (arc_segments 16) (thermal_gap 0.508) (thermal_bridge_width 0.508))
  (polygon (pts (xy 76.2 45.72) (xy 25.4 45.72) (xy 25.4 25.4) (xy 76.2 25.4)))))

